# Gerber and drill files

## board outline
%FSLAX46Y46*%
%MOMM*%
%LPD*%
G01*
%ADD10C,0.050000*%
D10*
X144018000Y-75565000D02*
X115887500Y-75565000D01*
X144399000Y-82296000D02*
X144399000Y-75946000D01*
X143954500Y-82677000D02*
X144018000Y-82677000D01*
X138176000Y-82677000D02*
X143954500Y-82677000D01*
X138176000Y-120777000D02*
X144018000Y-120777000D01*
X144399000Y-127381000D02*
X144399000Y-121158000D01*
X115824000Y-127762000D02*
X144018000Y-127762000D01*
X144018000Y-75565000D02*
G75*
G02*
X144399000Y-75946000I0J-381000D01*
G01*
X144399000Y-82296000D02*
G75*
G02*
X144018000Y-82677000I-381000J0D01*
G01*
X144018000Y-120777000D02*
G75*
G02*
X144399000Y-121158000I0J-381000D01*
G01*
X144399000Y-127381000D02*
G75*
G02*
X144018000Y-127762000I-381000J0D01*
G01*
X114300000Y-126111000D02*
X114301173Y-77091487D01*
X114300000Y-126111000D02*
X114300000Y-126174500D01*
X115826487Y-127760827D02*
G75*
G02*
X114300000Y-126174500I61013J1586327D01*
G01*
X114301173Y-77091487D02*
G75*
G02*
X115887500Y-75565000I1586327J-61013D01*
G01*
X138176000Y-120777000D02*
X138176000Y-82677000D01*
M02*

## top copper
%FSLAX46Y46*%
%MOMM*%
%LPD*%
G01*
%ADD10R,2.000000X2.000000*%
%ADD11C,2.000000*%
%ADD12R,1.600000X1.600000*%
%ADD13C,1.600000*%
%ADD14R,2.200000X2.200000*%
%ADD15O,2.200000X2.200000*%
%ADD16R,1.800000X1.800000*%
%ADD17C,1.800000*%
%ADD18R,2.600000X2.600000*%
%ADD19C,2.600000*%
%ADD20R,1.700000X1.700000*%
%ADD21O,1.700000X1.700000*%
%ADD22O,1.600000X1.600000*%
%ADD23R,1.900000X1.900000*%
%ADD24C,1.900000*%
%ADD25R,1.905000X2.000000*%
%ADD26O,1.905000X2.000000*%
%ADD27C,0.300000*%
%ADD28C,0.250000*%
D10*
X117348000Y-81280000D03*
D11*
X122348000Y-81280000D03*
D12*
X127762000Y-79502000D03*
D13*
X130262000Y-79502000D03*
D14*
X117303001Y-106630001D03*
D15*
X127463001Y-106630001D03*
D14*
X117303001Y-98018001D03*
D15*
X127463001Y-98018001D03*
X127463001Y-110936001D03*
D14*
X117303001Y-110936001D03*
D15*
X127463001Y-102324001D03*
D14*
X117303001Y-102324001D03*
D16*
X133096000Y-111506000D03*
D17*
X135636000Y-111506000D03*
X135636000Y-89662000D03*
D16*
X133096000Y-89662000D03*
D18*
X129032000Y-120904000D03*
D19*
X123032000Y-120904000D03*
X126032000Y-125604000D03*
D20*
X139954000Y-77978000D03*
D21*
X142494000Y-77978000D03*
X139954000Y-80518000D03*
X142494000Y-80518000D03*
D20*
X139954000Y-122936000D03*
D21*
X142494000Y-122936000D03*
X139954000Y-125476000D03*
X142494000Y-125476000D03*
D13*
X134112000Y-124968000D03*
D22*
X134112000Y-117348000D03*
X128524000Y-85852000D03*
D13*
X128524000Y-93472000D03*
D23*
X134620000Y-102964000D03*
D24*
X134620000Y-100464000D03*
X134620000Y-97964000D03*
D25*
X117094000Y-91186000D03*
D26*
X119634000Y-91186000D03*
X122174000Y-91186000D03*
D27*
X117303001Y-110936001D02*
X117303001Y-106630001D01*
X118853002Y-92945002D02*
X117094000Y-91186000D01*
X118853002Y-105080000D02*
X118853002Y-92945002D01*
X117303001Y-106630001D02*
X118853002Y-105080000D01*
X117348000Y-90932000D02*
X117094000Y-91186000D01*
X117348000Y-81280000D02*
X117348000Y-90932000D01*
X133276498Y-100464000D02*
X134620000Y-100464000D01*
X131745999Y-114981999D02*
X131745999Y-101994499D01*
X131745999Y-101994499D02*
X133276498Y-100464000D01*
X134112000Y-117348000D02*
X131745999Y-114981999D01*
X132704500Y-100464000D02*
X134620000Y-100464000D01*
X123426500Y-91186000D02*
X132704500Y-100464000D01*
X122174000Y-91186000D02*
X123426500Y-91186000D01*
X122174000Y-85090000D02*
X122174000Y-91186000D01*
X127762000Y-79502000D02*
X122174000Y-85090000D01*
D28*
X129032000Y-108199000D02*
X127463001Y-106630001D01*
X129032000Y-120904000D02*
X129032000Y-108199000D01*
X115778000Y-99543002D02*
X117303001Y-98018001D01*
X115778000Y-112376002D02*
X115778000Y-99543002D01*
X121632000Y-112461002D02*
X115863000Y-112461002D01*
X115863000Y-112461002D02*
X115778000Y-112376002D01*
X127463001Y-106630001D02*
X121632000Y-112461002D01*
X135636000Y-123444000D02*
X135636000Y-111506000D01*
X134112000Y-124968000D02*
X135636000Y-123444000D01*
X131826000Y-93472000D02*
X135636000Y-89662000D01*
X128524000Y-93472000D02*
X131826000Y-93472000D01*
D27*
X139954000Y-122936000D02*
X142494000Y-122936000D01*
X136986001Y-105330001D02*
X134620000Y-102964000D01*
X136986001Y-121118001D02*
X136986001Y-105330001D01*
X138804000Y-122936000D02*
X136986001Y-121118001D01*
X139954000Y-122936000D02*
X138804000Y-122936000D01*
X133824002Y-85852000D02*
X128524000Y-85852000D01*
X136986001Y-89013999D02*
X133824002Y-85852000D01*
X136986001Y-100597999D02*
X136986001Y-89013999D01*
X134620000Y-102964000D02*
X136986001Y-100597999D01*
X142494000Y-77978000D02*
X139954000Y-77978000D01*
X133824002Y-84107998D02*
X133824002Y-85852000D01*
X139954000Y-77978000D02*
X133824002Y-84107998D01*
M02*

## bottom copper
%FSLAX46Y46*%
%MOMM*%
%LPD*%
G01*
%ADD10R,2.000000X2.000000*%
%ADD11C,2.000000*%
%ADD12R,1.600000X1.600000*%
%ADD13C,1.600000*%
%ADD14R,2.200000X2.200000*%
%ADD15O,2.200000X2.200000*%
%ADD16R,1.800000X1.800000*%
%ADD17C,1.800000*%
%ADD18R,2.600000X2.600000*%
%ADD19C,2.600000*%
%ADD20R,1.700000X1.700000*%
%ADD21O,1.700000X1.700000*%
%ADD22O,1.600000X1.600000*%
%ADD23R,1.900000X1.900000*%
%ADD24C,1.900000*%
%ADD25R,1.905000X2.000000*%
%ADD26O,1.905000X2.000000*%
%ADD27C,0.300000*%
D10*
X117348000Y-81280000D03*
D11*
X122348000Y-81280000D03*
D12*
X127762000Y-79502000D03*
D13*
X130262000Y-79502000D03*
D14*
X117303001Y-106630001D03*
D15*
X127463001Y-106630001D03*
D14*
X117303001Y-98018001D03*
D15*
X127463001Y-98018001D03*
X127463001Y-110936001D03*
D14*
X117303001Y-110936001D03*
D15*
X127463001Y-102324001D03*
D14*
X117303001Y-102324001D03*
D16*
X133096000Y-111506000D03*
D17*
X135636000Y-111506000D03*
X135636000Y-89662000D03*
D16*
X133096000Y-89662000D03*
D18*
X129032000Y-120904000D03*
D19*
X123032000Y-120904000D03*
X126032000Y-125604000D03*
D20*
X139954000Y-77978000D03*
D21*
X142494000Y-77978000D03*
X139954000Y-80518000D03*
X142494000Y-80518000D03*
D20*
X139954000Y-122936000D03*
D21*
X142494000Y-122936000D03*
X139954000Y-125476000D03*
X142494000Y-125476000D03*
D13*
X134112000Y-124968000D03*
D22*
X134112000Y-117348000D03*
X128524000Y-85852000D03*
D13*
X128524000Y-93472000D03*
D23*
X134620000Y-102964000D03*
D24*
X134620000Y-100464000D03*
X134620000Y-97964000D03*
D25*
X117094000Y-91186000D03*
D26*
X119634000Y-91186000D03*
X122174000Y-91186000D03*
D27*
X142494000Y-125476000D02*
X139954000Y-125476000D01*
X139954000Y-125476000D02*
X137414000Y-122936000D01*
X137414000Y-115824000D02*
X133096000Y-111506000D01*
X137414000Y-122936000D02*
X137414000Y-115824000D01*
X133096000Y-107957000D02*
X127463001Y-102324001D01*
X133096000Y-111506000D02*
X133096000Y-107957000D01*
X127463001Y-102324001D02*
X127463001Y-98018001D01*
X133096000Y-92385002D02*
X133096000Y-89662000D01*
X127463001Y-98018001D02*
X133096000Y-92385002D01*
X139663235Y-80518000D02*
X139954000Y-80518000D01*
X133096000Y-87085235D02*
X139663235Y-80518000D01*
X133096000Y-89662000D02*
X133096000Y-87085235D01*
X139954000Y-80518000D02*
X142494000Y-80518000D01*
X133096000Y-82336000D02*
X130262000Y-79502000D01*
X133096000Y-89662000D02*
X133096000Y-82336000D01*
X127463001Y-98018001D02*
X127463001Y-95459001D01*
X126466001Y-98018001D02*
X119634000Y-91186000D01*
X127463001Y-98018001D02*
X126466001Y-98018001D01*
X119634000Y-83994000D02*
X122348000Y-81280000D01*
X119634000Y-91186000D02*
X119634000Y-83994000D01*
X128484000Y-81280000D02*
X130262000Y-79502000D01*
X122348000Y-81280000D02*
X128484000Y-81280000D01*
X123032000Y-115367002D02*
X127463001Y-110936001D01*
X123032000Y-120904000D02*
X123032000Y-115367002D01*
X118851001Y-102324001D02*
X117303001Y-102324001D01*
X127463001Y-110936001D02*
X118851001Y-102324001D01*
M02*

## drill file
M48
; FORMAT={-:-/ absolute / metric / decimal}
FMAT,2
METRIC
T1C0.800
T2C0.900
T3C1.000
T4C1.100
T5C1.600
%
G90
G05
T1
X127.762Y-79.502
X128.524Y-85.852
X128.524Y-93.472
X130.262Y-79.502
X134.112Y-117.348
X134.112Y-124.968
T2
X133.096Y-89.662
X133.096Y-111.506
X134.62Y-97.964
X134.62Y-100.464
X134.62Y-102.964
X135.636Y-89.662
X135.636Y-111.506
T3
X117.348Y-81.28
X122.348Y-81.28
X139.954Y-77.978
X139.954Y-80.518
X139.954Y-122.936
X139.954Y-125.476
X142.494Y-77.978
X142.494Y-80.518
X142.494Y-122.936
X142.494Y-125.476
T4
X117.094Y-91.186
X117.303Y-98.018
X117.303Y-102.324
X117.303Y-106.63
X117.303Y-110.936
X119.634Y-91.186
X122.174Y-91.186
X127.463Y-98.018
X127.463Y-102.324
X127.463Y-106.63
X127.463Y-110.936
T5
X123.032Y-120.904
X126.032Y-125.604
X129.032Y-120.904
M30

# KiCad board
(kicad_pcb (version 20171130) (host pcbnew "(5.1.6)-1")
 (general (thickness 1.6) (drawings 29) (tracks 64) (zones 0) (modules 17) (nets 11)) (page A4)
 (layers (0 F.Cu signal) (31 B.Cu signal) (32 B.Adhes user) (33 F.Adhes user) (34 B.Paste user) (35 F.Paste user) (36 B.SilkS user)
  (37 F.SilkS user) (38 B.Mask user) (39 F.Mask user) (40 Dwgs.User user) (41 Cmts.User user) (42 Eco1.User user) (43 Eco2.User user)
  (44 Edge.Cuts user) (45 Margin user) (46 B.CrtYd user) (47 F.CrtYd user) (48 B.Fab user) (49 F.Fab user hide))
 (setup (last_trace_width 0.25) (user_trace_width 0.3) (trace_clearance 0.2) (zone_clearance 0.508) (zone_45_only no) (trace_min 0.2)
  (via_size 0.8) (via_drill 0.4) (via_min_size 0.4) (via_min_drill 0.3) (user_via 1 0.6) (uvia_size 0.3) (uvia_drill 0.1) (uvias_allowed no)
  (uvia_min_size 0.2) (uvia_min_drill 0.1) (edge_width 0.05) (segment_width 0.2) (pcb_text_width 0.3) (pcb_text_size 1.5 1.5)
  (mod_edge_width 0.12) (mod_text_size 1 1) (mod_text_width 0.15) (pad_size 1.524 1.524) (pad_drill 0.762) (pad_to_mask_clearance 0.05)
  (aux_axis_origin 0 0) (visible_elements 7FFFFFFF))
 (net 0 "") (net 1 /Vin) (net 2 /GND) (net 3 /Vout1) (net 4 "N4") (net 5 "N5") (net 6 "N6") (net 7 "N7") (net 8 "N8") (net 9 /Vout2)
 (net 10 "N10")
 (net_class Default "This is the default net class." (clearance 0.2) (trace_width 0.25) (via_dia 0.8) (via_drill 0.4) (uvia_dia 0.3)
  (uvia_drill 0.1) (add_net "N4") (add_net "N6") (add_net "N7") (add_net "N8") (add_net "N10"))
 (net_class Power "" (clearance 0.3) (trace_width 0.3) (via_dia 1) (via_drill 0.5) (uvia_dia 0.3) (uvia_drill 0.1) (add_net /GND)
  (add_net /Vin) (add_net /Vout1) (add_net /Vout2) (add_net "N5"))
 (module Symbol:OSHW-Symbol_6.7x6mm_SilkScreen (layer B.Cu) (at 121.158 86.106 270)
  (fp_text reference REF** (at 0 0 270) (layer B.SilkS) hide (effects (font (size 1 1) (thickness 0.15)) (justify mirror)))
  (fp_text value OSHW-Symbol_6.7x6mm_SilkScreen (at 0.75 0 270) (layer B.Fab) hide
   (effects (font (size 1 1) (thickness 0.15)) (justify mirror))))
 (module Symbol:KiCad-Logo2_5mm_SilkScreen (layer B.Cu) (at 122.682 104.394 270)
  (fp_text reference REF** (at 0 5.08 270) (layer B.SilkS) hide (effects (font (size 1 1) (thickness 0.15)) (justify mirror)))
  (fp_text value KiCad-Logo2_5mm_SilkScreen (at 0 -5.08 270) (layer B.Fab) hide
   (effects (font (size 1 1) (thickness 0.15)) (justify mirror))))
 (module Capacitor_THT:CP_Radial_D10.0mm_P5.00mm (layer F.Cu) (at 117.348 81.28)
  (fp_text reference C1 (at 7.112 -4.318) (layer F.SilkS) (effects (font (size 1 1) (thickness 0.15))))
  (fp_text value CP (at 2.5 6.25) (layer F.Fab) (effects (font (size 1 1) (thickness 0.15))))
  (pad 1 thru_hole rect (at 0 0) (size 2 2) (drill 1) (layers *.Cu *.Mask) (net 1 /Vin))
  (pad 2 thru_hole circle (at 5 0) (size 2 2) (drill 1) (layers *.Cu *.Mask) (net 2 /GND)))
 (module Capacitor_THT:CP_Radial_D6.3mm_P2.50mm (layer F.Cu) (at 127.762 79.502)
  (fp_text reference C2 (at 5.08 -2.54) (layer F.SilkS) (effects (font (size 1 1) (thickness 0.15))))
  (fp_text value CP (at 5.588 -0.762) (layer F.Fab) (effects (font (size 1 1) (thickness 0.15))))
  (pad 1 thru_hole rect (at 0 0) (size 1.6 1.6) (drill 0.8) (layers *.Cu *.Mask) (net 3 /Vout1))
  (pad 2 thru_hole circle (at 2.5 0) (size 1.6 1.6) (drill 0.8) (layers *.Cu *.Mask) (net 2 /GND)))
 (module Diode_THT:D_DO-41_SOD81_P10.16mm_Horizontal (layer F.Cu) (at 117.303001 106.630001)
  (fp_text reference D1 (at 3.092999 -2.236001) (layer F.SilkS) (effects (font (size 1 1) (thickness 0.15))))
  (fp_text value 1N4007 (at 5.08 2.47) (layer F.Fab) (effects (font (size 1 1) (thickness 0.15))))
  (pad 1 thru_hole rect (at 0 0) (size 2.2 2.2) (drill 1.1) (layers *.Cu *.Mask) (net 1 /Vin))
  (pad 2 thru_hole oval (at 10.16 0) (size 2.2 2.2) (drill 1.1) (layers *.Cu *.Mask) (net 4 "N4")))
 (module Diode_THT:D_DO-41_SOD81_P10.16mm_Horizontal (layer F.Cu) (at 117.303001 98.018001)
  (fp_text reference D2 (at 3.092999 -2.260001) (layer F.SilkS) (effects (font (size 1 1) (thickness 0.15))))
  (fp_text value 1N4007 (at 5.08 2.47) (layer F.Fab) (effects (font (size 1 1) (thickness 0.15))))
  (pad 1 thru_hole rect (at 0 0) (size 2.2 2.2) (drill 1.1) (layers *.Cu *.Mask) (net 4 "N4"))
  (pad 2 thru_hole oval (at 10.16 0) (size 2.2 2.2) (drill 1.1) (layers *.Cu *.Mask) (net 2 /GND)))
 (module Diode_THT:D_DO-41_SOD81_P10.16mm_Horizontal (layer F.Cu) (at 117.303001 110.936001)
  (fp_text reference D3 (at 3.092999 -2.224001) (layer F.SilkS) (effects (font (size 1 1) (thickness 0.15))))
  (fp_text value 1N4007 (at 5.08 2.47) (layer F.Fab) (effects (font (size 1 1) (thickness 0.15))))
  (pad 2 thru_hole oval (at 10.16 0) (size 2.2 2.2) (drill 1.1) (layers *.Cu *.Mask) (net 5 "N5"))
  (pad 1 thru_hole rect (at 0 0) (size 2.2 2.2) (drill 1.1) (layers *.Cu *.Mask) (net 1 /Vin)))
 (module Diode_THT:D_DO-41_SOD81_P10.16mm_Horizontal (layer F.Cu) (at 117.303001 102.324001)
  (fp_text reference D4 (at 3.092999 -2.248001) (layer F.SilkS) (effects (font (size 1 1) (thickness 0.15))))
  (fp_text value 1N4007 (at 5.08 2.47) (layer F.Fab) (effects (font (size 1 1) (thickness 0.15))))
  (pad 2 thru_hole oval (at 10.16 0) (size 2.2 2.2) (drill 1.1) (layers *.Cu *.Mask) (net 2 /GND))
  (pad 1 thru_hole rect (at 0 0) (size 2.2 2.2) (drill 1.1) (layers *.Cu *.Mask) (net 5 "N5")))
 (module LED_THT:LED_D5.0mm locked (layer F.Cu) (at 133.096 111.506)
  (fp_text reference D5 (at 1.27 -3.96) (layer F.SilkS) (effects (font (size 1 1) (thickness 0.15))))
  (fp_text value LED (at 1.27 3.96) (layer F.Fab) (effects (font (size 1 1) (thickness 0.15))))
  (pad 1 thru_hole rect (at 0 0) (size 1.8 1.8) (drill 0.9) (layers *.Cu *.Mask) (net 2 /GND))
  (pad 2 thru_hole circle (at 2.54 0) (size 1.8 1.8) (drill 0.9) (layers *.Cu *.Mask) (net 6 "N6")))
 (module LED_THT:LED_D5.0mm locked (layer F.Cu) (at 133.096 89.662)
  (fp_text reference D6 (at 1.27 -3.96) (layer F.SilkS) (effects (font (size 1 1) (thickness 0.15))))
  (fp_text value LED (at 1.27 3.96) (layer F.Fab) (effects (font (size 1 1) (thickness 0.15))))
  (pad 2 thru_hole circle (at 2.54 0) (size 1.8 1.8) (drill 0.9) (layers *.Cu *.Mask) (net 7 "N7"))
  (pad 1 thru_hole rect (at 0 0) (size 1.8 1.8) (drill 0.9) (layers *.Cu *.Mask) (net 2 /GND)))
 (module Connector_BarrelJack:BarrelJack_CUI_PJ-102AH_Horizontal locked (layer F.Cu) (at 129.032 120.904 270)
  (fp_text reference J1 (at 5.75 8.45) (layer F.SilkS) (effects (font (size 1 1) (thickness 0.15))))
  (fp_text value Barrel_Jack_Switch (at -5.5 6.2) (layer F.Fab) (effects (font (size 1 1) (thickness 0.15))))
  (pad 1 thru_hole rect (at 0 0 270) (size 2.6 2.6) (drill 1.6) (layers *.Cu *.Mask) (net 4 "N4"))
  (pad 2 thru_hole circle (at 0 6 270) (size 2.6 2.6) (drill 1.6) (layers *.Cu *.Mask) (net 5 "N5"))
  (pad 3 thru_hole circle (at 4.7 3 270) (size 2.6 2.6) (drill 1.6) (layers *.Cu *.Mask) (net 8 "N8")))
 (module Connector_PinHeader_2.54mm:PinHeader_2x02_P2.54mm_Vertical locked (layer F.Cu) (at 139.954 77.978)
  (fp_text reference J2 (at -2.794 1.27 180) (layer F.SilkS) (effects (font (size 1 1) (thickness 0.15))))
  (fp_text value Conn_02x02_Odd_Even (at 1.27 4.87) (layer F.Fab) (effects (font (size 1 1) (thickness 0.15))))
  (pad 1 thru_hole rect (at 0 0) (size 1.7 1.7) (drill 1) (layers *.Cu *.Mask) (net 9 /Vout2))
  (pad 2 thru_hole oval (at 2.54 0) (size 1.7 1.7) (drill 1) (layers *.Cu *.Mask) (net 9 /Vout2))
  (pad 3 thru_hole oval (at 0 2.54) (size 1.7 1.7) (drill 1) (layers *.Cu *.Mask) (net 2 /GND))
  (pad 4 thru_hole oval (at 2.54 2.54) (size 1.7 1.7) (drill 1) (layers *.Cu *.Mask) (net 2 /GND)))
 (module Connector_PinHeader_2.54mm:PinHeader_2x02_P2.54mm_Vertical (layer F.Cu) (at 139.954 122.936)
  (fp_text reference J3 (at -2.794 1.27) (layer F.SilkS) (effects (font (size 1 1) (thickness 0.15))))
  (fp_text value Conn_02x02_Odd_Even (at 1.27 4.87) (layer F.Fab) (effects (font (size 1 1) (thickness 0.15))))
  (pad 1 thru_hole rect (at 0 0) (size 1.7 1.7) (drill 1) (layers *.Cu *.Mask) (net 9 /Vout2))
  (pad 2 thru_hole oval (at 2.54 0) (size 1.7 1.7) (drill 1) (layers *.Cu *.Mask) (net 9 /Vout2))
  (pad 3 thru_hole oval (at 0 2.54) (size 1.7 1.7) (drill 1) (layers *.Cu *.Mask) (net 2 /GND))
  (pad 4 thru_hole oval (at 2.54 2.54) (size 1.7 1.7) (drill 1) (layers *.Cu *.Mask) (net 2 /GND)))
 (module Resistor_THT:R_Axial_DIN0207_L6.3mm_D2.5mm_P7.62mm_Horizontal (layer F.Cu) (at 134.112 124.968 90)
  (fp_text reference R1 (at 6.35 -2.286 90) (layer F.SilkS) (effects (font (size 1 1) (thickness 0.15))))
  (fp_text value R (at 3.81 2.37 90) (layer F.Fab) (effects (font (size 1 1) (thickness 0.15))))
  (pad 1 thru_hole circle (at 0 0 90) (size 1.6 1.6) (drill 0.8) (layers *.Cu *.Mask) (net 6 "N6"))
  (pad 2 thru_hole oval (at 7.62 0 90) (size 1.6 1.6) (drill 0.8) (layers *.Cu *.Mask) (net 3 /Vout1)))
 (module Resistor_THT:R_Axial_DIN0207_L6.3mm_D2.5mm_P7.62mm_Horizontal (layer F.Cu) (at 128.524 93.472 90)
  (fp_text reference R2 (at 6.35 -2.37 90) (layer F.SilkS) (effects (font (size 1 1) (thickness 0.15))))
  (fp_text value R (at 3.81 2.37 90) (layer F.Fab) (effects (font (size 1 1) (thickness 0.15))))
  (pad 2 thru_hole oval (at 7.62 0 90) (size 1.6 1.6) (drill 0.8) (layers *.Cu *.Mask) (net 9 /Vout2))
  (pad 1 thru_hole circle (at 0 0 90) (size 1.6 1.6) (drill 0.8) (layers *.Cu *.Mask) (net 7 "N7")))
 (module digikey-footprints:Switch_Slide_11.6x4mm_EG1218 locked (layer F.Cu) (at 134.62 102.964 90)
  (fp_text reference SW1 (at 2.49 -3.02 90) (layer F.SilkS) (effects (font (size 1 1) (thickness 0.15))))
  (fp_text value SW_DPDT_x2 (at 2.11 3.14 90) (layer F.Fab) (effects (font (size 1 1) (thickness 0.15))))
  (pad 1 thru_hole rect (at 0 0 90) (size 1.9 1.9) (drill 0.9) (layers *.Cu *.Mask) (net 9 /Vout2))
  (pad 2 thru_hole circle (at 2.5 0 90) (size 1.9 1.9) (drill 0.9) (layers *.Cu *.Mask) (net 3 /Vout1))
  (pad 3 thru_hole circle (at 5 0 90) (size 1.9 1.9) (drill 0.9) (layers *.Cu *.Mask) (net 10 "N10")))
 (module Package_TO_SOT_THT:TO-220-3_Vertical (layer F.Cu) (at 117.094 91.186)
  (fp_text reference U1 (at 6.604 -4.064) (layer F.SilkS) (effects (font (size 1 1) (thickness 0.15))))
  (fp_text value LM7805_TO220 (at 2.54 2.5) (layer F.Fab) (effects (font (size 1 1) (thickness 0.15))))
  (pad 1 thru_hole rect (at 0 0) (size 1.905 2) (drill 1.1) (layers *.Cu *.Mask) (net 1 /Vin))
  (pad 2 thru_hole oval (at 2.54 0) (size 1.905 2) (drill 1.1) (layers *.Cu *.Mask) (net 2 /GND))
  (pad 3 thru_hole oval (at 5.08 0) (size 1.905 2) (drill 1.1) (layers *.Cu *.Mask) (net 3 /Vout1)))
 (gr_line (start 144.018 75.565) (end 115.8875 75.565) (layer Edge.Cuts) (width 0.05))
 (gr_line (start 144.399 82.296) (end 144.399 75.946) (layer Edge.Cuts) (width 0.05))
 (gr_line (start 143.9545 82.677) (end 144.018 82.677) (layer Edge.Cuts) (width 0.05))
 (gr_line (start 138.176 82.677) (end 143.9545 82.677) (layer Edge.Cuts) (width 0.05))
 (gr_line (start 138.176 120.777) (end 144.018 120.777) (layer Edge.Cuts) (width 0.05))
 (gr_line (start 144.399 127.381) (end 144.399 121.158) (layer Edge.Cuts) (width 0.05))
 (gr_line (start 115.824 127.762) (end 144.018 127.762) (layer Edge.Cuts) (width 0.05))
 (gr_arc (start 144.018 75.946) (end 144.399 75.946) (angle -90) (layer Edge.Cuts) (width 0.05))
 (gr_arc (start 144.018 82.296) (end 144.018 82.677) (angle -90) (layer Edge.Cuts) (width 0.05))
 (gr_arc (start 144.018 121.158) (end 144.399 121.158) (angle -90) (layer Edge.Cuts) (width 0.05))
 (gr_arc (start 144.018 127.381) (end 144.018 127.762) (angle -90) (layer Edge.Cuts) (width 0.05))
 (gr_line (start 114.3 126.111) (end 114.301173 77.091487) (layer Edge.Cuts) (width 0.05))
 (gr_line (start 114.3 126.111) (end 114.3 126.1745) (layer Edge.Cuts) (width 0.05))
 (gr_arc (start 115.8875 126.1745) (end 114.3 126.1745) (angle -87.79740184) (layer Edge.Cuts) (width 0.05))
 (gr_arc (start 115.8875 77.1525) (end 115.8875 75.565) (angle -87.79740184) (layer Edge.Cuts) (width 0.05))
 (gr_line (start 138.176 120.777) (end 138.176 82.677) (layer Edge.Cuts) (width 0.05))
 (segment (start 117.303001 110.936001) (end 117.303001 106.630001) (width 0.3) (layer F.Cu) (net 1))
 (segment (start 118.853002 92.945002) (end 117.094 91.186) (width 0.3) (layer F.Cu) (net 1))
 (segment (start 118.853002 105.08) (end 118.853002 92.945002) (width 0.3) (layer F.Cu) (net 1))
 (segment (start 117.303001 106.630001) (end 118.853002 105.08) (width 0.3) (layer F.Cu) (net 1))
 (segment (start 117.348 90.932) (end 117.094 91.186) (width 0.3) (layer F.Cu) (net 1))
 (segment (start 117.348 81.28) (end 117.348 90.932) (width 0.3) (layer F.Cu) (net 1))
 (segment (start 142.494 125.476) (end 139.954 125.476) (width 0.3) (layer B.Cu) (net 2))
 (segment (start 139.954 125.476) (end 137.414 122.936) (width 0.3) (layer B.Cu) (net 2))
 (segment (start 137.414 115.824) (end 133.096 111.506) (width 0.3) (layer B.Cu) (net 2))
 (segment (start 137.414 122.936) (end 137.414 115.824) (width 0.3) (layer B.Cu) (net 2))
 (segment (start 133.096 107.957) (end 127.463001 102.324001) (width 0.3) (layer B.Cu) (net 2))
 (segment (start 133.096 111.506) (end 133.096 107.957) (width 0.3) (layer B.Cu) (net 2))
 (segment (start 127.463001 102.324001) (end 127.463001 98.018001) (width 0.3) (layer B.Cu) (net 2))
 (segment (start 133.096 92.385002) (end 133.096 89.662) (width 0.3) (layer B.Cu) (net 2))
 (segment (start 127.463001 98.018001) (end 133.096 92.385002) (width 0.3) (layer B.Cu) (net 2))
 (segment (start 139.663235 80.518) (end 139.954 80.518) (width 0.3) (layer B.Cu) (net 2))
 (segment (start 133.096 87.085235) (end 139.663235 80.518) (width 0.3) (layer B.Cu) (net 2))
 (segment (start 133.096 89.662) (end 133.096 87.085235) (width 0.3) (layer B.Cu) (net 2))
 (segment (start 139.954 80.518) (end 142.494 80.518) (width 0.3) (layer B.Cu) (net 2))
 (segment (start 133.096 82.336) (end 130.262 79.502) (width 0.3) (layer B.Cu) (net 2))
 (segment (start 133.096 89.662) (end 133.096 82.336) (width 0.3) (layer B.Cu) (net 2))
 (segment (start 127.463001 98.018001) (end 127.463001 95.459001) (width 0.3) (layer B.Cu) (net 2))
 (segment (start 126.466001 98.018001) (end 119.634 91.186) (width 0.3) (layer B.Cu) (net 2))
 (segment (start 127.463001 98.018001) (end 126.466001 98.018001) (width 0.3) (layer B.Cu) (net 2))
 (segment (start 119.634 83.994) (end 122.348 81.28) (width 0.3) (layer B.Cu) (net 2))
 (segment (start 119.634 91.186) (end 119.634 83.994) (width 0.3) (layer B.Cu) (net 2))
 (segment (start 128.484 81.28) (end 130.262 79.502) (width 0.3) (layer B.Cu) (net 2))
 (segment (start 122.348 81.28) (end 128.484 81.28) (width 0.3) (layer B.Cu) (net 2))
 (segment (start 133.276498 100.464) (end 134.62 100.464) (width 0.3) (layer F.Cu) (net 3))
 (segment (start 131.745999 114.981999) (end 131.745999 101.994499) (width 0.3) (layer F.Cu) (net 3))
 (segment (start 131.745999 101.994499) (end 133.276498 100.464) (width 0.3) (layer F.Cu) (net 3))
 (segment (start 134.112 117.348) (end 131.745999 114.981999) (width 0.3) (layer F.Cu) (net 3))
 (segment (start 132.7045 100.464) (end 134.62 100.464) (width 0.3) (layer F.Cu) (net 3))
 (segment (start 123.4265 91.186) (end 132.7045 100.464) (width 0.3) (layer F.Cu) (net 3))
 (segment (start 122.174 91.186) (end 123.4265 91.186) (width 0.3) (layer F.Cu) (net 3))
 (segment (start 122.174 85.09) (end 122.174 91.186) (width 0.3) (layer F.Cu) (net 3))
 (segment (start 127.762 79.502) (end 122.174 85.09) (width 0.3) (layer F.Cu) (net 3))
 (segment (start 129.032 108.199) (end 127.463001 106.630001) (width 0.25) (layer F.Cu) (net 4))
 (segment (start 129.032 120.904) (end 129.032 108.199) (width 0.25) (layer F.Cu) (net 4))
 (segment (start 115.778 99.543002) (end 117.303001 98.018001) (width 0.25) (layer F.Cu) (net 4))
 (segment (start 115.778 112.376002) (end 115.778 99.543002) (width 0.25) (layer F.Cu) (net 4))
 (segment (start 121.632 112.461002) (end 115.863 112.461002) (width 0.25) (layer F.Cu) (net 4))
 (segment (start 115.863 112.461002) (end 115.778 112.376002) (width 0.25) (layer F.Cu) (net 4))
 (segment (start 127.463001 106.630001) (end 121.632 112.461002) (width 0.25) (layer F.Cu) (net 4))
 (segment (start 123.032 115.367002) (end 127.463001 110.936001) (width 0.3) (layer B.Cu) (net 5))
 (segment (start 123.032 120.904) (end 123.032 115.367002) (width 0.3) (layer B.Cu) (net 5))
 (segment (start 118.851001 102.324001) (end 117.303001 102.324001) (width 0.3) (layer B.Cu) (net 5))
 (segment (start 127.463001 110.936001) (end 118.851001 102.324001) (width 0.3) (layer B.Cu) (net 5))
 (segment (start 135.636 123.444) (end 135.636 111.506) (width 0.25) (layer F.Cu) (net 6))
 (segment (start 134.112 124.968) (end 135.636 123.444) (width 0.25) (layer F.Cu) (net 6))
 (segment (start 131.826 93.472) (end 135.636 89.662) (width 0.25) (layer F.Cu) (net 7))
 (segment (start 128.524 93.472) (end 131.826 93.472) (width 0.25) (layer F.Cu) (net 7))
 (segment (start 139.954 122.936) (end 142.494 122.936) (width 0.3) (layer F.Cu) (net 9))
 (segment (start 136.986001 105.330001) (end 134.62 102.964) (width 0.3) (layer F.Cu) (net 9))
 (segment (start 136.986001 121.118001) (end 136.986001 105.330001) (width 0.3) (layer F.Cu) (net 9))
 (segment (start 138.804 122.936) (end 136.986001 121.118001) (width 0.3) (layer F.Cu) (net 9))
 (segment (start 139.954 122.936) (end 138.804 122.936) (width 0.3) (layer F.Cu) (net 9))
 (segment (start 133.824002 85.852) (end 128.524 85.852) (width 0.3) (layer F.Cu) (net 9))
 (segment (start 136.986001 89.013999) (end 133.824002 85.852) (width 0.3) (layer F.Cu) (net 9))
 (segment (start 136.986001 100.597999) (end 136.986001 89.013999) (width 0.3) (layer F.Cu) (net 9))
 (segment (start 134.62 102.964) (end 136.986001 100.597999) (width 0.3) (layer F.Cu) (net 9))
 (segment (start 142.494 77.978) (end 139.954 77.978) (width 0.3) (layer F.Cu) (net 9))
 (segment (start 133.824002 84.107998) (end 133.824002 85.852) (width 0.3) (layer F.Cu) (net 9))
 (segment (start 139.954 77.978) (end 133.824002 84.107998) (width 0.3) (layer F.Cu) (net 9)))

